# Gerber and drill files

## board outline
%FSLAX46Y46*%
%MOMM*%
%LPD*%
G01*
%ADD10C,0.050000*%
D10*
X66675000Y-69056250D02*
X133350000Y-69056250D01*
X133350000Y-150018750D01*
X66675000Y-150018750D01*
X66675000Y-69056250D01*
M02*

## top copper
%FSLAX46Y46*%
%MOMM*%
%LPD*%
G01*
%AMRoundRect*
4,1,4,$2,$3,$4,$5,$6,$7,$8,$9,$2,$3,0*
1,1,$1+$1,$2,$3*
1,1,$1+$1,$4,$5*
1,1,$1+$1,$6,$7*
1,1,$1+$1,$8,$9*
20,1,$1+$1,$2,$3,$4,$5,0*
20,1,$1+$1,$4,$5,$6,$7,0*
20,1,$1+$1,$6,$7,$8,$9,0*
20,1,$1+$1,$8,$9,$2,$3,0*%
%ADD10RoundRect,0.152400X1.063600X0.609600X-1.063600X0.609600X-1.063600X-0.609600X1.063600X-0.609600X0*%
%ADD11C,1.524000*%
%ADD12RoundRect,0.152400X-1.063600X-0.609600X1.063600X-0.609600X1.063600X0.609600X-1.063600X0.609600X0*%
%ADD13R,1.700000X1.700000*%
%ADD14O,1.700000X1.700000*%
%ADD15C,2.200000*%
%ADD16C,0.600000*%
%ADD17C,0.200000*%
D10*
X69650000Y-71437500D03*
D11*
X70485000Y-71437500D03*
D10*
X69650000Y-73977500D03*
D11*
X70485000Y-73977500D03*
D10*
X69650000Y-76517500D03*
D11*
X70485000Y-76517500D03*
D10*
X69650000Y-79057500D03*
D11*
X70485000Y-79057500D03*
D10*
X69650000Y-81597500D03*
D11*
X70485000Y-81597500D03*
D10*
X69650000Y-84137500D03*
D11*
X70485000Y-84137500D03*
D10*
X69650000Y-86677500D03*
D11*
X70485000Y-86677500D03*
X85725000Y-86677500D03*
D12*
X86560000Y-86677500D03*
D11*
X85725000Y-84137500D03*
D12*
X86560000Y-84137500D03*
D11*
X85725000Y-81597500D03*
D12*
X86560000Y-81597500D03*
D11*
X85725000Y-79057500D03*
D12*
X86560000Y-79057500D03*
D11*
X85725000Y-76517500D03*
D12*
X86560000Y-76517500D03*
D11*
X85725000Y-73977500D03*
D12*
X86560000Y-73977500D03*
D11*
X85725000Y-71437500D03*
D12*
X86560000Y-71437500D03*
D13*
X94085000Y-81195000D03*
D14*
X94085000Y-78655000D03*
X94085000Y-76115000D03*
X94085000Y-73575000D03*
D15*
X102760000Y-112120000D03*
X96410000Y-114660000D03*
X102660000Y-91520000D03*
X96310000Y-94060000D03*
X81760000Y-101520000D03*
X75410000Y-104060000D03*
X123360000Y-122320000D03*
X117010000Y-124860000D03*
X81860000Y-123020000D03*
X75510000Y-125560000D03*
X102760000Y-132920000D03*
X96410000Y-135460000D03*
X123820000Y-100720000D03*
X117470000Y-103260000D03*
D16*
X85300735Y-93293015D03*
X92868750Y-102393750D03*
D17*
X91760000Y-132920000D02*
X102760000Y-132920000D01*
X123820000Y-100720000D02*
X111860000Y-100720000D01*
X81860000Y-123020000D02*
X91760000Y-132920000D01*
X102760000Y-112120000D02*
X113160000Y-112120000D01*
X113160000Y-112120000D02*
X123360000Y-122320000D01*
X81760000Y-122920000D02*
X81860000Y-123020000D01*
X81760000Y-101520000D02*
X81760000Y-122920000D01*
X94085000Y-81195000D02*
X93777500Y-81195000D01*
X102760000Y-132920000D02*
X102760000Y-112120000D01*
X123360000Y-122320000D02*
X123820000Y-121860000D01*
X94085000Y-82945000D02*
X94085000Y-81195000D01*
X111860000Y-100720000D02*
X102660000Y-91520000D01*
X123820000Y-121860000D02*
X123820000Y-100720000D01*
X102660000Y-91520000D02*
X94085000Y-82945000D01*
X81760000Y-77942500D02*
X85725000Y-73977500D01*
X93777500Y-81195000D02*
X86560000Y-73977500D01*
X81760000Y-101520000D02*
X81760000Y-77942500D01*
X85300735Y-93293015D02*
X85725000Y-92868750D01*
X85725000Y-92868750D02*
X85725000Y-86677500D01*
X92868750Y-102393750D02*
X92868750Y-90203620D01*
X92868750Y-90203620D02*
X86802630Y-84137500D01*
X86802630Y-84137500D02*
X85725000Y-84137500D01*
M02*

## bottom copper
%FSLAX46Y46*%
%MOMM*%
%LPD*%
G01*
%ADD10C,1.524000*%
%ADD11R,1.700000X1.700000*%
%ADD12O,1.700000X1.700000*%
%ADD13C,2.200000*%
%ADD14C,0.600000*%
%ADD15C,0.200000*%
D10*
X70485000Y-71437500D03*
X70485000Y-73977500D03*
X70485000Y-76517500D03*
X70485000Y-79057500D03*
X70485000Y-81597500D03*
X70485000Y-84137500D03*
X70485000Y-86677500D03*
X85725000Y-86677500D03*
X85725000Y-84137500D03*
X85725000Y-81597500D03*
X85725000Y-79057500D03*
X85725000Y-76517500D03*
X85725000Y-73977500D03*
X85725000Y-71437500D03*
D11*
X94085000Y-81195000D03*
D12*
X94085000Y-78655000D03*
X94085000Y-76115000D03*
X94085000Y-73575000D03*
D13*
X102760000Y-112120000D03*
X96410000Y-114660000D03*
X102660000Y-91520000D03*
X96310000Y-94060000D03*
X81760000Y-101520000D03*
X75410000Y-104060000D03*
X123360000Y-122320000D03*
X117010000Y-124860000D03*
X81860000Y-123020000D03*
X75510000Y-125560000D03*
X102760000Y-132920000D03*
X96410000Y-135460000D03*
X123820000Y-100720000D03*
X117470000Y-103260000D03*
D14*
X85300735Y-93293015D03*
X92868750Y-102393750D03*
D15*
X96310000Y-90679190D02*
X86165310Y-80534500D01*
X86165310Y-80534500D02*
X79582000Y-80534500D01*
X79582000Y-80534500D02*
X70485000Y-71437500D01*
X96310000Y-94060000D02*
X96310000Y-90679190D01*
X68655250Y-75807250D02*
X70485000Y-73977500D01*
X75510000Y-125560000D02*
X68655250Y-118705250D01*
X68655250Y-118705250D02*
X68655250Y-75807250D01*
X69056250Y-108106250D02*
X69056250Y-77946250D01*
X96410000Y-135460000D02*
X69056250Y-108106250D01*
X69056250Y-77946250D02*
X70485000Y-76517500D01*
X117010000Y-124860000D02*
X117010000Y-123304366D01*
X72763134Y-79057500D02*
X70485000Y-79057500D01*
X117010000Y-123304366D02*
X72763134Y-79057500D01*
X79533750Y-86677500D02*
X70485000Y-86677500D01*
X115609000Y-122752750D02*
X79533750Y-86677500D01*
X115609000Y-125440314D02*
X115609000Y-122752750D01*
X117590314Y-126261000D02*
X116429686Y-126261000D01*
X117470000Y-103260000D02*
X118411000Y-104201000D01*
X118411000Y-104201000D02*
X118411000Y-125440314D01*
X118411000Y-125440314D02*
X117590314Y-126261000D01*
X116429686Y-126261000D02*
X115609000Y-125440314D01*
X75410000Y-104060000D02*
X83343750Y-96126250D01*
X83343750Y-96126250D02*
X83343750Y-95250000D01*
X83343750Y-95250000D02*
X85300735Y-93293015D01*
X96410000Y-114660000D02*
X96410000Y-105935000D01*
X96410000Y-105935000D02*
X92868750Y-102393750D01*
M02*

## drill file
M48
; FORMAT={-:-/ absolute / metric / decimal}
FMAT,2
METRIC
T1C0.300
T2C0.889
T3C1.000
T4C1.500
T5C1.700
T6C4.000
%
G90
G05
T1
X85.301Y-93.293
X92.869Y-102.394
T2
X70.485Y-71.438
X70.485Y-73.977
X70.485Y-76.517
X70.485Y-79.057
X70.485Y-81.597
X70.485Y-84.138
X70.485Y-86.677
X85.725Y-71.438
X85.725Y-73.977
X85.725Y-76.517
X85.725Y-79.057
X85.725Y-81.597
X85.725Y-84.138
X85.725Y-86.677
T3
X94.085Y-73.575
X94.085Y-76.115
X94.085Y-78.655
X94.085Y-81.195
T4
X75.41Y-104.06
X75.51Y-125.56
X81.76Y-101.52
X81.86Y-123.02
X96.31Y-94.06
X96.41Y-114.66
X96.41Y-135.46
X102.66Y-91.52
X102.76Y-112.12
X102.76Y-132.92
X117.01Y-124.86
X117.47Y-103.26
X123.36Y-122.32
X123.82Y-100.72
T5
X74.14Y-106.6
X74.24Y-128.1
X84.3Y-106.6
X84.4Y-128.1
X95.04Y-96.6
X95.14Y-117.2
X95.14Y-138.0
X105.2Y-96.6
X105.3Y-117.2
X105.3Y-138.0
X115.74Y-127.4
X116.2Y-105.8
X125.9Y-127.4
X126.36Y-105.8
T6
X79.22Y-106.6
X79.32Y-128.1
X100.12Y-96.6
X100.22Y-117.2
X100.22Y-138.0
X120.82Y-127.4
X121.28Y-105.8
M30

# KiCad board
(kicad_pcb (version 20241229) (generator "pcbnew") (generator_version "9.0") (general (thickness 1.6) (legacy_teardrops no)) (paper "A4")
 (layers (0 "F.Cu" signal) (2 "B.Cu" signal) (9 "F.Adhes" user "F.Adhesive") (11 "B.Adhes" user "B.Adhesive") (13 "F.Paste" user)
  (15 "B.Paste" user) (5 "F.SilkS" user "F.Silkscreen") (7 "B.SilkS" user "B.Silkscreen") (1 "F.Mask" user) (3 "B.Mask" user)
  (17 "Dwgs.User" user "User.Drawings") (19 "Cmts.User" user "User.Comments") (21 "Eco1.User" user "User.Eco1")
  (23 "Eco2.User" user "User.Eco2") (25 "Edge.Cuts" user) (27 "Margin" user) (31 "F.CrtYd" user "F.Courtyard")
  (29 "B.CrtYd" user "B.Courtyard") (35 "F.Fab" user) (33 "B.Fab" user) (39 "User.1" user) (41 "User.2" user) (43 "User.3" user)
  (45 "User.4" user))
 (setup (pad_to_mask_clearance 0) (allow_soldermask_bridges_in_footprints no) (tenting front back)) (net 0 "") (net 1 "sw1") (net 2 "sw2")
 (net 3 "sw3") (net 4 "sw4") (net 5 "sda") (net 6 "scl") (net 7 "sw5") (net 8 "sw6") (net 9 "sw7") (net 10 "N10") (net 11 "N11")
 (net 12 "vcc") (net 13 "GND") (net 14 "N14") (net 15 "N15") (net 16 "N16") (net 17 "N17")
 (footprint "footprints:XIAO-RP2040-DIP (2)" (layer "F.Cu") (at 78.105 79.0575)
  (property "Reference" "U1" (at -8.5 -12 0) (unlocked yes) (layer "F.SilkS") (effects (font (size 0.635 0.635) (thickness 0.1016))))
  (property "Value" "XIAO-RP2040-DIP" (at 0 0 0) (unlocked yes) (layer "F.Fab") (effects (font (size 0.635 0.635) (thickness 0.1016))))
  (pad "1" smd roundrect (at -8.455 -7.62 180) (size 2.432 1.524) (layers "F.Cu" "F.Mask") (roundrect_rratio 0.1) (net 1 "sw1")
   (thermal_bridge_angle 45))
  (pad "1" thru_hole circle (at -7.62 -7.62 180) (size 1.524 1.524) (drill 0.889) (layers "*.Cu" "*.Mask") (remove_unused_layers no)
   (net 1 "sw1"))
  (pad "2" smd roundrect (at -8.455 -5.08 180) (size 2.432 1.524) (layers "F.Cu" "F.Mask") (roundrect_rratio 0.1) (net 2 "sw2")
   (thermal_bridge_angle 45))
  (pad "2" thru_hole circle (at -7.62 -5.08 180) (size 1.524 1.524) (drill 0.889) (layers "*.Cu" "*.Mask") (remove_unused_layers no)
   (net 2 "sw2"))
  (pad "3" smd roundrect (at -8.455 -2.54 180) (size 2.432 1.524) (layers "F.Cu" "F.Mask") (roundrect_rratio 0.1) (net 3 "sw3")
   (thermal_bridge_angle 45))
  (pad "3" thru_hole circle (at -7.62 -2.54 180) (size 1.524 1.524) (drill 0.889) (layers "*.Cu" "*.Mask") (remove_unused_layers no)
   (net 3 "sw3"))
  (pad "4" smd roundrect (at -8.455 0 180) (size 2.432 1.524) (layers "F.Cu" "F.Mask") (roundrect_rratio 0.1) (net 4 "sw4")
   (thermal_bridge_angle 45))
  (pad "4" thru_hole circle (at -7.62 0 180) (size 1.524 1.524) (drill 0.889) (layers "*.Cu" "*.Mask") (remove_unused_layers no)
   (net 4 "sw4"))
  (pad "5" smd roundrect (at -8.455 2.54 180) (size 2.432 1.524) (layers "F.Cu" "F.Mask") (roundrect_rratio 0.1) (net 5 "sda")
   (thermal_bridge_angle 45))
  (pad "5" thru_hole circle (at -7.62 2.54 180) (size 1.524 1.524) (drill 0.889) (layers "*.Cu" "*.Mask") (remove_unused_layers no)
   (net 5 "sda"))
  (pad "6" smd roundrect (at -8.455 5.08 180) (size 2.432 1.524) (layers "F.Cu" "F.Mask") (roundrect_rratio 0.1) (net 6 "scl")
   (thermal_bridge_angle 45))
  (pad "6" thru_hole circle (at -7.62 5.08 180) (size 1.524 1.524) (drill 0.889) (layers "*.Cu" "*.Mask") (remove_unused_layers no)
   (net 6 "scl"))
  (pad "7" smd roundrect (at -8.455 7.62 180) (size 2.432 1.524) (layers "F.Cu" "F.Mask") (roundrect_rratio 0.1) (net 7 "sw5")
   (thermal_bridge_angle 45))
  (pad "7" thru_hole circle (at -7.62 7.62 180) (size 1.524 1.524) (drill 0.889) (layers "*.Cu" "*.Mask") (remove_unused_layers no)
   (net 7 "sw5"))
  (pad "8" thru_hole circle (at 7.62 7.62) (size 1.524 1.524) (drill 0.889) (layers "*.Cu" "*.Mask") (remove_unused_layers no) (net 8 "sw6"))
  (pad "8" smd roundrect (at 8.455 7.62) (size 2.432 1.524) (layers "F.Cu" "F.Mask") (roundrect_rratio 0.1) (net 8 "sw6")
   (thermal_bridge_angle 45))
  (pad "9" thru_hole circle (at 7.62 5.08) (size 1.524 1.524) (drill 0.889) (layers "*.Cu" "*.Mask") (remove_unused_layers no) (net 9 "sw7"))
  (pad "9" smd roundrect (at 8.455 5.08) (size 2.432 1.524) (layers "F.Cu" "F.Mask") (roundrect_rratio 0.1) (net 9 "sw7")
   (thermal_bridge_angle 45))
  (pad "10" thru_hole circle (at 7.62 2.54) (size 1.524 1.524) (drill 0.889) (layers "*.Cu" "*.Mask") (remove_unused_layers no)
   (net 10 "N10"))
  (pad "10" smd roundrect (at 8.455 2.54) (size 2.432 1.524) (layers "F.Cu" "F.Mask") (roundrect_rratio 0.1) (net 10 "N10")
   (thermal_bridge_angle 45))
  (pad "11" thru_hole circle (at 7.62 0) (size 1.524 1.524) (drill 0.889) (layers "*.Cu" "*.Mask") (remove_unused_layers no) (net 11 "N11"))
  (pad "11" smd roundrect (at 8.455 0) (size 2.432 1.524) (layers "F.Cu" "F.Mask") (roundrect_rratio 0.1) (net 11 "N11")
   (thermal_bridge_angle 45))
  (pad "12" thru_hole circle (at 7.62 -2.54) (size 1.524 1.524) (drill 0.889) (layers "*.Cu" "*.Mask") (remove_unused_layers no)
   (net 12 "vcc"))
  (pad "12" smd roundrect (at 8.455 -2.54) (size 2.432 1.524) (layers "F.Cu" "F.Mask") (roundrect_rratio 0.1) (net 12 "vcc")
   (thermal_bridge_angle 45))
  (pad "13" thru_hole circle (at 7.62 -5.08) (size 1.524 1.524) (drill 0.889) (layers "*.Cu" "*.Mask") (remove_unused_layers no)
   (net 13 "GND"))
  (pad "13" smd roundrect (at 8.455 -5.08) (size 2.432 1.524) (layers "F.Cu" "F.Mask") (roundrect_rratio 0.1) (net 13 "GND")
   (thermal_bridge_angle 45))
  (pad "14" thru_hole circle (at 7.62 -7.62) (size 1.524 1.524) (drill 0.889) (layers "*.Cu" "*.Mask") (remove_unused_layers no)
   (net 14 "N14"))
  (pad "14" smd roundrect (at 8.455 -7.62) (size 2.432 1.524) (layers "F.Cu" "F.Mask") (roundrect_rratio 0.1) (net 14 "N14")
   (thermal_bridge_angle 45)))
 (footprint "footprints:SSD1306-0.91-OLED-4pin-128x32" (layer "F.Cu") (at 130.585 83.385 180)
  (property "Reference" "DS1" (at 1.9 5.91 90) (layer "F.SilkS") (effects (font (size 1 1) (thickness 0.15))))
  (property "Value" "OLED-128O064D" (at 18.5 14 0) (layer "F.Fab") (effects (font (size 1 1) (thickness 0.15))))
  (pad "1" thru_hole rect (at 36.5 2.19 180) (size 1.7 1.7) (drill 1) (layers "*.Cu" "*.Mask") (remove_unused_layers no) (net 13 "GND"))
  (pad "2" thru_hole oval (at 36.5 4.73 180) (size 1.7 1.7) (drill 1) (layers "*.Cu" "*.Mask") (remove_unused_layers no) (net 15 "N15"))
  (pad "3" thru_hole oval (at 36.5 7.27 180) (size 1.7 1.7) (drill 1) (layers "*.Cu" "*.Mask") (remove_unused_layers no) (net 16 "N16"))
  (pad "4" thru_hole oval (at 36.5 9.81 180) (size 1.7 1.7) (drill 1) (layers "*.Cu" "*.Mask") (remove_unused_layers no) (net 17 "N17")))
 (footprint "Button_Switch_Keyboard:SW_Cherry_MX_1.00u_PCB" (layer "F.Cu") (at 102.76 112.12)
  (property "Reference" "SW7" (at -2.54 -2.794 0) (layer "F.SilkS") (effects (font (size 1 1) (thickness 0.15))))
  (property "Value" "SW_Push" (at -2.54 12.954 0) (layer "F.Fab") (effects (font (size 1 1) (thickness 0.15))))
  (pad "" np_thru_hole circle (at -7.62 5.08) (size 1.7 1.7) (drill 1.7) (layers "*.Cu" "*.Mask"))
  (pad "" np_thru_hole circle (at -2.54 5.08) (size 4 4) (drill 4) (layers "*.Cu" "*.Mask"))
  (pad "" np_thru_hole circle (at 2.54 5.08) (size 1.7 1.7) (drill 1.7) (layers "*.Cu" "*.Mask"))
  (pad "1" thru_hole circle (at 0 0) (size 2.2 2.2) (drill 1.5) (layers "*.Cu" "*.Mask") (remove_unused_layers no) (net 13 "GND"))
  (pad "2" thru_hole circle (at -6.35 2.54) (size 2.2 2.2) (drill 1.5) (layers "*.Cu" "*.Mask") (remove_unused_layers no) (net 9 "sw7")))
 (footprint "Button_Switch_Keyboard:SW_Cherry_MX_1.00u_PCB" (layer "F.Cu") (at 102.66 91.52)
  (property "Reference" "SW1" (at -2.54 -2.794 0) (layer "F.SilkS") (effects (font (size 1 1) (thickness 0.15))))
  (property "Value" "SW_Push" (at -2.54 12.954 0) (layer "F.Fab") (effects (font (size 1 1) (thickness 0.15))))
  (pad "" np_thru_hole circle (at -7.62 5.08) (size 1.7 1.7) (drill 1.7) (layers "*.Cu" "*.Mask"))
  (pad "" np_thru_hole circle (at -2.54 5.08) (size 4 4) (drill 4) (layers "*.Cu" "*.Mask"))
  (pad "" np_thru_hole circle (at 2.54 5.08) (size 1.7 1.7) (drill 1.7) (layers "*.Cu" "*.Mask"))
  (pad "1" thru_hole circle (at 0 0) (size 2.2 2.2) (drill 1.5) (layers "*.Cu" "*.Mask") (remove_unused_layers no) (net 13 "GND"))
  (pad "2" thru_hole circle (at -6.35 2.54) (size 2.2 2.2) (drill 1.5) (layers "*.Cu" "*.Mask") (remove_unused_layers no) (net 1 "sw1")))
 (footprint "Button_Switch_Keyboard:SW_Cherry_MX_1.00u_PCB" (layer "F.Cu") (at 81.76 101.52)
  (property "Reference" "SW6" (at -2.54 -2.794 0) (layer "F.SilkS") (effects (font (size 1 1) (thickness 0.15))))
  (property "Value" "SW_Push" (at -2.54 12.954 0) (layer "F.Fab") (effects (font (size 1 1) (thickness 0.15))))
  (pad "" np_thru_hole circle (at -7.62 5.08) (size 1.7 1.7) (drill 1.7) (layers "*.Cu" "*.Mask"))
  (pad "" np_thru_hole circle (at -2.54 5.08) (size 4 4) (drill 4) (layers "*.Cu" "*.Mask"))
  (pad "" np_thru_hole circle (at 2.54 5.08) (size 1.7 1.7) (drill 1.7) (layers "*.Cu" "*.Mask"))
  (pad "1" thru_hole circle (at 0 0) (size 2.2 2.2) (drill 1.5) (layers "*.Cu" "*.Mask") (remove_unused_layers no) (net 13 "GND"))
  (pad "2" thru_hole circle (at -6.35 2.54) (size 2.2 2.2) (drill 1.5) (layers "*.Cu" "*.Mask") (remove_unused_layers no) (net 8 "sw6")))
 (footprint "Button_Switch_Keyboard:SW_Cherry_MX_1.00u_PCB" (layer "F.Cu") (at 123.36 122.32)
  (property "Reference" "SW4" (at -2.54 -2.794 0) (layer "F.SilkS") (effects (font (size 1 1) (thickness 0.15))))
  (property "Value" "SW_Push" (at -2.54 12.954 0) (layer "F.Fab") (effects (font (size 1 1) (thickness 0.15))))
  (pad "" np_thru_hole circle (at -7.62 5.08) (size 1.7 1.7) (drill 1.7) (layers "*.Cu" "*.Mask"))
  (pad "" np_thru_hole circle (at -2.54 5.08) (size 4 4) (drill 4) (layers "*.Cu" "*.Mask"))
  (pad "" np_thru_hole circle (at 2.54 5.08) (size 1.7 1.7) (drill 1.7) (layers "*.Cu" "*.Mask"))
  (pad "1" thru_hole circle (at 0 0) (size 2.2 2.2) (drill 1.5) (layers "*.Cu" "*.Mask") (remove_unused_layers no) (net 13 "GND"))
  (pad "2" thru_hole circle (at -6.35 2.54) (size 2.2 2.2) (drill 1.5) (layers "*.Cu" "*.Mask") (remove_unused_layers no) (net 4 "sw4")))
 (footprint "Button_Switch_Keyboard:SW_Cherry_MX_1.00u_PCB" (layer "F.Cu") (at 81.86 123.02)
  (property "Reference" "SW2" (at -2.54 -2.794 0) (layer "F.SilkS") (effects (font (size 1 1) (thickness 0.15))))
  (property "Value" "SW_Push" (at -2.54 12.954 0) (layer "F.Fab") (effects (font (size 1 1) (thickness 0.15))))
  (pad "" np_thru_hole circle (at -7.62 5.08) (size 1.7 1.7) (drill 1.7) (layers "*.Cu" "*.Mask"))
  (pad "" np_thru_hole circle (at -2.54 5.08) (size 4 4) (drill 4) (layers "*.Cu" "*.Mask"))
  (pad "" np_thru_hole circle (at 2.54 5.08) (size 1.7 1.7) (drill 1.7) (layers "*.Cu" "*.Mask"))
  (pad "1" thru_hole circle (at 0 0) (size 2.2 2.2) (drill 1.5) (layers "*.Cu" "*.Mask") (remove_unused_layers no) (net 13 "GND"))
  (pad "2" thru_hole circle (at -6.35 2.54) (size 2.2 2.2) (drill 1.5) (layers "*.Cu" "*.Mask") (remove_unused_layers no) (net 2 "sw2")))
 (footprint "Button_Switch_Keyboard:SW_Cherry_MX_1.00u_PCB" (layer "F.Cu") (at 102.76 132.92)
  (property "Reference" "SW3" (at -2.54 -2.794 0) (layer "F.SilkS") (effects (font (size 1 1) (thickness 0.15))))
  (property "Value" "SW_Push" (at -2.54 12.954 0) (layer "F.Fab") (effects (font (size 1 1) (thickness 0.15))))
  (pad "" np_thru_hole circle (at -7.62 5.08) (size 1.7 1.7) (drill 1.7) (layers "*.Cu" "*.Mask"))
  (pad "" np_thru_hole circle (at -2.54 5.08) (size 4 4) (drill 4) (layers "*.Cu" "*.Mask"))
  (pad "" np_thru_hole circle (at 2.54 5.08) (size 1.7 1.7) (drill 1.7) (layers "*.Cu" "*.Mask"))
  (pad "1" thru_hole circle (at 0 0) (size 2.2 2.2) (drill 1.5) (layers "*.Cu" "*.Mask") (remove_unused_layers no) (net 13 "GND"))
  (pad "2" thru_hole circle (at -6.35 2.54) (size 2.2 2.2) (drill 1.5) (layers "*.Cu" "*.Mask") (remove_unused_layers no) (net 3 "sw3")))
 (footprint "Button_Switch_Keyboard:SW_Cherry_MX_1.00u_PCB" (layer "F.Cu") (at 123.82 100.72)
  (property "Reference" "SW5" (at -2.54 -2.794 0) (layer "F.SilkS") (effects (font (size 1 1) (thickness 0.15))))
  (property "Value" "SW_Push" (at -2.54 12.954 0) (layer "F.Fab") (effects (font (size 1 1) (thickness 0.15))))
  (pad "" np_thru_hole circle (at -7.62 5.08) (size 1.7 1.7) (drill 1.7) (layers "*.Cu" "*.Mask"))
  (pad "" np_thru_hole circle (at -2.54 5.08) (size 4 4) (drill 4) (layers "*.Cu" "*.Mask"))
  (pad "" np_thru_hole circle (at 2.54 5.08) (size 1.7 1.7) (drill 1.7) (layers "*.Cu" "*.Mask"))
  (pad "1" thru_hole circle (at 0 0) (size 2.2 2.2) (drill 1.5) (layers "*.Cu" "*.Mask") (remove_unused_layers no) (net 13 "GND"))
  (pad "2" thru_hole circle (at -6.35 2.54) (size 2.2 2.2) (drill 1.5) (layers "*.Cu" "*.Mask") (remove_unused_layers no) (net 7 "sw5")))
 (gr_rect (start 66.675 69.05625) (end 133.35 150.01875) (stroke (width 0.05) (type default)) (fill no) (layer "Edge.Cuts"))
 (segment (start 91.76 132.92) (end 102.76 132.92) (width 0.2) (layer "F.Cu") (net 13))
 (segment (start 123.82 100.72) (end 111.86 100.72) (width 0.2) (layer "F.Cu") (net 13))
 (segment (start 81.86 123.02) (end 91.76 132.92) (width 0.2) (layer "F.Cu") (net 13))
 (segment (start 102.76 112.12) (end 113.16 112.12) (width 0.2) (layer "F.Cu") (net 13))
 (segment (start 113.16 112.12) (end 123.36 122.32) (width 0.2) (layer "F.Cu") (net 13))
 (segment (start 81.76 122.92) (end 81.86 123.02) (width 0.2) (layer "F.Cu") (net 13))
 (segment (start 81.76 101.52) (end 81.76 122.92) (width 0.2) (layer "F.Cu") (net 13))
 (segment (start 94.085 81.195) (end 93.7775 81.195) (width 0.2) (layer "F.Cu") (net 13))
 (segment (start 102.76 132.92) (end 102.76 112.12) (width 0.2) (layer "F.Cu") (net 13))
 (segment (start 123.36 122.32) (end 123.82 121.86) (width 0.2) (layer "F.Cu") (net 13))
 (segment (start 94.085 82.945) (end 94.085 81.195) (width 0.2) (layer "F.Cu") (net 13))
 (segment (start 111.86 100.72) (end 102.66 91.52) (width 0.2) (layer "F.Cu") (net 13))
 (segment (start 123.82 121.86) (end 123.82 100.72) (width 0.2) (layer "F.Cu") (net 13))
 (segment (start 102.66 91.52) (end 94.085 82.945) (width 0.2) (layer "F.Cu") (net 13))
 (segment (start 81.76 77.9425) (end 85.725 73.9775) (width 0.2) (layer "F.Cu") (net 13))
 (segment (start 93.7775 81.195) (end 86.56 73.9775) (width 0.2) (layer "F.Cu") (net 13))
 (segment (start 81.76 101.52) (end 81.76 77.9425) (width 0.2) (layer "F.Cu") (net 13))
 (segment (start 96.31 90.67919) (end 86.16531 80.5345) (width 0.2) (layer "B.Cu") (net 1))
 (segment (start 86.16531 80.5345) (end 79.582 80.5345) (width 0.2) (layer "B.Cu") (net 1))
 (segment (start 79.582 80.5345) (end 70.485 71.4375) (width 0.2) (layer "B.Cu") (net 1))
 (segment (start 96.31 94.06) (end 96.31 90.67919) (width 0.2) (layer "B.Cu") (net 1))
 (segment (start 68.65525 75.80725) (end 70.485 73.9775) (width 0.2) (layer "B.Cu") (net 2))
 (segment (start 75.51 125.56) (end 68.65525 118.70525) (width 0.2) (layer "B.Cu") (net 2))
 (segment (start 68.65525 118.70525) (end 68.65525 75.80725) (width 0.2) (layer "B.Cu") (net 2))
 (segment (start 69.05625 108.10625) (end 69.05625 77.94625) (width 0.2) (layer "B.Cu") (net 3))
 (segment (start 96.41 135.46) (end 69.05625 108.10625) (width 0.2) (layer "B.Cu") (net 3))
 (segment (start 69.05625 77.94625) (end 70.485 76.5175) (width 0.2) (layer "B.Cu") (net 3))
 (segment (start 117.01 124.86) (end 117.01 123.304366) (width 0.2) (layer "B.Cu") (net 4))
 (segment (start 72.763134 79.0575) (end 70.485 79.0575) (width 0.2) (layer "B.Cu") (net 4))
 (segment (start 117.01 123.304366) (end 72.763134 79.0575) (width 0.2) (layer "B.Cu") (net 4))
 (segment (start 79.53375 86.6775) (end 70.485 86.6775) (width 0.2) (layer "B.Cu") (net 7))
 (segment (start 115.609 122.75275) (end 79.53375 86.6775) (width 0.2) (layer "B.Cu") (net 7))
 (segment (start 115.609 125.440314) (end 115.609 122.75275) (width 0.2) (layer "B.Cu") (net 7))
 (segment (start 117.590314 126.261) (end 116.429686 126.261) (width 0.2) (layer "B.Cu") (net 7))
 (segment (start 117.47 103.26) (end 118.411 104.201) (width 0.2) (layer "B.Cu") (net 7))
 (segment (start 118.411 104.201) (end 118.411 125.440314) (width 0.2) (layer "B.Cu") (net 7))
 (segment (start 118.411 125.440314) (end 117.590314 126.261) (width 0.2) (layer "B.Cu") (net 7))
 (segment (start 116.429686 126.261) (end 115.609 125.440314) (width 0.2) (layer "B.Cu") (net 7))
 (segment (start 85.300735 93.293015) (end 85.725 92.86875) (width 0.2) (layer "F.Cu") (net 8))
 (segment (start 85.725 92.86875) (end 85.725 86.6775) (width 0.2) (layer "F.Cu") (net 8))
 (via (at 85.300735 93.293015) (size 0.6) (drill 0.3) (layers "F.Cu" "B.Cu") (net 8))
 (segment (start 75.41 104.06) (end 83.34375 96.12625) (width 0.2) (layer "B.Cu") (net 8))
 (segment (start 83.34375 96.12625) (end 83.34375 95.25) (width 0.2) (layer "B.Cu") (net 8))
 (segment (start 83.34375 95.25) (end 85.300735 93.293015) (width 0.2) (layer "B.Cu") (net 8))
 (segment (start 92.86875 102.39375) (end 92.86875 90.20362) (width 0.2) (layer "F.Cu") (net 9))
 (segment (start 92.86875 90.20362) (end 86.80263 84.1375) (width 0.2) (layer "F.Cu") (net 9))
 (segment (start 86.80263 84.1375) (end 85.725 84.1375) (width 0.2) (layer "F.Cu") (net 9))
 (via (at 92.86875 102.39375) (size 0.6) (drill 0.3) (layers "F.Cu" "B.Cu") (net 9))
 (segment (start 96.41 114.66) (end 96.41 105.935) (width 0.2) (layer "B.Cu") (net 9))
 (segment (start 96.41 105.935) (end 92.86875 102.39375) (width 0.2) (layer "B.Cu") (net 9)))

